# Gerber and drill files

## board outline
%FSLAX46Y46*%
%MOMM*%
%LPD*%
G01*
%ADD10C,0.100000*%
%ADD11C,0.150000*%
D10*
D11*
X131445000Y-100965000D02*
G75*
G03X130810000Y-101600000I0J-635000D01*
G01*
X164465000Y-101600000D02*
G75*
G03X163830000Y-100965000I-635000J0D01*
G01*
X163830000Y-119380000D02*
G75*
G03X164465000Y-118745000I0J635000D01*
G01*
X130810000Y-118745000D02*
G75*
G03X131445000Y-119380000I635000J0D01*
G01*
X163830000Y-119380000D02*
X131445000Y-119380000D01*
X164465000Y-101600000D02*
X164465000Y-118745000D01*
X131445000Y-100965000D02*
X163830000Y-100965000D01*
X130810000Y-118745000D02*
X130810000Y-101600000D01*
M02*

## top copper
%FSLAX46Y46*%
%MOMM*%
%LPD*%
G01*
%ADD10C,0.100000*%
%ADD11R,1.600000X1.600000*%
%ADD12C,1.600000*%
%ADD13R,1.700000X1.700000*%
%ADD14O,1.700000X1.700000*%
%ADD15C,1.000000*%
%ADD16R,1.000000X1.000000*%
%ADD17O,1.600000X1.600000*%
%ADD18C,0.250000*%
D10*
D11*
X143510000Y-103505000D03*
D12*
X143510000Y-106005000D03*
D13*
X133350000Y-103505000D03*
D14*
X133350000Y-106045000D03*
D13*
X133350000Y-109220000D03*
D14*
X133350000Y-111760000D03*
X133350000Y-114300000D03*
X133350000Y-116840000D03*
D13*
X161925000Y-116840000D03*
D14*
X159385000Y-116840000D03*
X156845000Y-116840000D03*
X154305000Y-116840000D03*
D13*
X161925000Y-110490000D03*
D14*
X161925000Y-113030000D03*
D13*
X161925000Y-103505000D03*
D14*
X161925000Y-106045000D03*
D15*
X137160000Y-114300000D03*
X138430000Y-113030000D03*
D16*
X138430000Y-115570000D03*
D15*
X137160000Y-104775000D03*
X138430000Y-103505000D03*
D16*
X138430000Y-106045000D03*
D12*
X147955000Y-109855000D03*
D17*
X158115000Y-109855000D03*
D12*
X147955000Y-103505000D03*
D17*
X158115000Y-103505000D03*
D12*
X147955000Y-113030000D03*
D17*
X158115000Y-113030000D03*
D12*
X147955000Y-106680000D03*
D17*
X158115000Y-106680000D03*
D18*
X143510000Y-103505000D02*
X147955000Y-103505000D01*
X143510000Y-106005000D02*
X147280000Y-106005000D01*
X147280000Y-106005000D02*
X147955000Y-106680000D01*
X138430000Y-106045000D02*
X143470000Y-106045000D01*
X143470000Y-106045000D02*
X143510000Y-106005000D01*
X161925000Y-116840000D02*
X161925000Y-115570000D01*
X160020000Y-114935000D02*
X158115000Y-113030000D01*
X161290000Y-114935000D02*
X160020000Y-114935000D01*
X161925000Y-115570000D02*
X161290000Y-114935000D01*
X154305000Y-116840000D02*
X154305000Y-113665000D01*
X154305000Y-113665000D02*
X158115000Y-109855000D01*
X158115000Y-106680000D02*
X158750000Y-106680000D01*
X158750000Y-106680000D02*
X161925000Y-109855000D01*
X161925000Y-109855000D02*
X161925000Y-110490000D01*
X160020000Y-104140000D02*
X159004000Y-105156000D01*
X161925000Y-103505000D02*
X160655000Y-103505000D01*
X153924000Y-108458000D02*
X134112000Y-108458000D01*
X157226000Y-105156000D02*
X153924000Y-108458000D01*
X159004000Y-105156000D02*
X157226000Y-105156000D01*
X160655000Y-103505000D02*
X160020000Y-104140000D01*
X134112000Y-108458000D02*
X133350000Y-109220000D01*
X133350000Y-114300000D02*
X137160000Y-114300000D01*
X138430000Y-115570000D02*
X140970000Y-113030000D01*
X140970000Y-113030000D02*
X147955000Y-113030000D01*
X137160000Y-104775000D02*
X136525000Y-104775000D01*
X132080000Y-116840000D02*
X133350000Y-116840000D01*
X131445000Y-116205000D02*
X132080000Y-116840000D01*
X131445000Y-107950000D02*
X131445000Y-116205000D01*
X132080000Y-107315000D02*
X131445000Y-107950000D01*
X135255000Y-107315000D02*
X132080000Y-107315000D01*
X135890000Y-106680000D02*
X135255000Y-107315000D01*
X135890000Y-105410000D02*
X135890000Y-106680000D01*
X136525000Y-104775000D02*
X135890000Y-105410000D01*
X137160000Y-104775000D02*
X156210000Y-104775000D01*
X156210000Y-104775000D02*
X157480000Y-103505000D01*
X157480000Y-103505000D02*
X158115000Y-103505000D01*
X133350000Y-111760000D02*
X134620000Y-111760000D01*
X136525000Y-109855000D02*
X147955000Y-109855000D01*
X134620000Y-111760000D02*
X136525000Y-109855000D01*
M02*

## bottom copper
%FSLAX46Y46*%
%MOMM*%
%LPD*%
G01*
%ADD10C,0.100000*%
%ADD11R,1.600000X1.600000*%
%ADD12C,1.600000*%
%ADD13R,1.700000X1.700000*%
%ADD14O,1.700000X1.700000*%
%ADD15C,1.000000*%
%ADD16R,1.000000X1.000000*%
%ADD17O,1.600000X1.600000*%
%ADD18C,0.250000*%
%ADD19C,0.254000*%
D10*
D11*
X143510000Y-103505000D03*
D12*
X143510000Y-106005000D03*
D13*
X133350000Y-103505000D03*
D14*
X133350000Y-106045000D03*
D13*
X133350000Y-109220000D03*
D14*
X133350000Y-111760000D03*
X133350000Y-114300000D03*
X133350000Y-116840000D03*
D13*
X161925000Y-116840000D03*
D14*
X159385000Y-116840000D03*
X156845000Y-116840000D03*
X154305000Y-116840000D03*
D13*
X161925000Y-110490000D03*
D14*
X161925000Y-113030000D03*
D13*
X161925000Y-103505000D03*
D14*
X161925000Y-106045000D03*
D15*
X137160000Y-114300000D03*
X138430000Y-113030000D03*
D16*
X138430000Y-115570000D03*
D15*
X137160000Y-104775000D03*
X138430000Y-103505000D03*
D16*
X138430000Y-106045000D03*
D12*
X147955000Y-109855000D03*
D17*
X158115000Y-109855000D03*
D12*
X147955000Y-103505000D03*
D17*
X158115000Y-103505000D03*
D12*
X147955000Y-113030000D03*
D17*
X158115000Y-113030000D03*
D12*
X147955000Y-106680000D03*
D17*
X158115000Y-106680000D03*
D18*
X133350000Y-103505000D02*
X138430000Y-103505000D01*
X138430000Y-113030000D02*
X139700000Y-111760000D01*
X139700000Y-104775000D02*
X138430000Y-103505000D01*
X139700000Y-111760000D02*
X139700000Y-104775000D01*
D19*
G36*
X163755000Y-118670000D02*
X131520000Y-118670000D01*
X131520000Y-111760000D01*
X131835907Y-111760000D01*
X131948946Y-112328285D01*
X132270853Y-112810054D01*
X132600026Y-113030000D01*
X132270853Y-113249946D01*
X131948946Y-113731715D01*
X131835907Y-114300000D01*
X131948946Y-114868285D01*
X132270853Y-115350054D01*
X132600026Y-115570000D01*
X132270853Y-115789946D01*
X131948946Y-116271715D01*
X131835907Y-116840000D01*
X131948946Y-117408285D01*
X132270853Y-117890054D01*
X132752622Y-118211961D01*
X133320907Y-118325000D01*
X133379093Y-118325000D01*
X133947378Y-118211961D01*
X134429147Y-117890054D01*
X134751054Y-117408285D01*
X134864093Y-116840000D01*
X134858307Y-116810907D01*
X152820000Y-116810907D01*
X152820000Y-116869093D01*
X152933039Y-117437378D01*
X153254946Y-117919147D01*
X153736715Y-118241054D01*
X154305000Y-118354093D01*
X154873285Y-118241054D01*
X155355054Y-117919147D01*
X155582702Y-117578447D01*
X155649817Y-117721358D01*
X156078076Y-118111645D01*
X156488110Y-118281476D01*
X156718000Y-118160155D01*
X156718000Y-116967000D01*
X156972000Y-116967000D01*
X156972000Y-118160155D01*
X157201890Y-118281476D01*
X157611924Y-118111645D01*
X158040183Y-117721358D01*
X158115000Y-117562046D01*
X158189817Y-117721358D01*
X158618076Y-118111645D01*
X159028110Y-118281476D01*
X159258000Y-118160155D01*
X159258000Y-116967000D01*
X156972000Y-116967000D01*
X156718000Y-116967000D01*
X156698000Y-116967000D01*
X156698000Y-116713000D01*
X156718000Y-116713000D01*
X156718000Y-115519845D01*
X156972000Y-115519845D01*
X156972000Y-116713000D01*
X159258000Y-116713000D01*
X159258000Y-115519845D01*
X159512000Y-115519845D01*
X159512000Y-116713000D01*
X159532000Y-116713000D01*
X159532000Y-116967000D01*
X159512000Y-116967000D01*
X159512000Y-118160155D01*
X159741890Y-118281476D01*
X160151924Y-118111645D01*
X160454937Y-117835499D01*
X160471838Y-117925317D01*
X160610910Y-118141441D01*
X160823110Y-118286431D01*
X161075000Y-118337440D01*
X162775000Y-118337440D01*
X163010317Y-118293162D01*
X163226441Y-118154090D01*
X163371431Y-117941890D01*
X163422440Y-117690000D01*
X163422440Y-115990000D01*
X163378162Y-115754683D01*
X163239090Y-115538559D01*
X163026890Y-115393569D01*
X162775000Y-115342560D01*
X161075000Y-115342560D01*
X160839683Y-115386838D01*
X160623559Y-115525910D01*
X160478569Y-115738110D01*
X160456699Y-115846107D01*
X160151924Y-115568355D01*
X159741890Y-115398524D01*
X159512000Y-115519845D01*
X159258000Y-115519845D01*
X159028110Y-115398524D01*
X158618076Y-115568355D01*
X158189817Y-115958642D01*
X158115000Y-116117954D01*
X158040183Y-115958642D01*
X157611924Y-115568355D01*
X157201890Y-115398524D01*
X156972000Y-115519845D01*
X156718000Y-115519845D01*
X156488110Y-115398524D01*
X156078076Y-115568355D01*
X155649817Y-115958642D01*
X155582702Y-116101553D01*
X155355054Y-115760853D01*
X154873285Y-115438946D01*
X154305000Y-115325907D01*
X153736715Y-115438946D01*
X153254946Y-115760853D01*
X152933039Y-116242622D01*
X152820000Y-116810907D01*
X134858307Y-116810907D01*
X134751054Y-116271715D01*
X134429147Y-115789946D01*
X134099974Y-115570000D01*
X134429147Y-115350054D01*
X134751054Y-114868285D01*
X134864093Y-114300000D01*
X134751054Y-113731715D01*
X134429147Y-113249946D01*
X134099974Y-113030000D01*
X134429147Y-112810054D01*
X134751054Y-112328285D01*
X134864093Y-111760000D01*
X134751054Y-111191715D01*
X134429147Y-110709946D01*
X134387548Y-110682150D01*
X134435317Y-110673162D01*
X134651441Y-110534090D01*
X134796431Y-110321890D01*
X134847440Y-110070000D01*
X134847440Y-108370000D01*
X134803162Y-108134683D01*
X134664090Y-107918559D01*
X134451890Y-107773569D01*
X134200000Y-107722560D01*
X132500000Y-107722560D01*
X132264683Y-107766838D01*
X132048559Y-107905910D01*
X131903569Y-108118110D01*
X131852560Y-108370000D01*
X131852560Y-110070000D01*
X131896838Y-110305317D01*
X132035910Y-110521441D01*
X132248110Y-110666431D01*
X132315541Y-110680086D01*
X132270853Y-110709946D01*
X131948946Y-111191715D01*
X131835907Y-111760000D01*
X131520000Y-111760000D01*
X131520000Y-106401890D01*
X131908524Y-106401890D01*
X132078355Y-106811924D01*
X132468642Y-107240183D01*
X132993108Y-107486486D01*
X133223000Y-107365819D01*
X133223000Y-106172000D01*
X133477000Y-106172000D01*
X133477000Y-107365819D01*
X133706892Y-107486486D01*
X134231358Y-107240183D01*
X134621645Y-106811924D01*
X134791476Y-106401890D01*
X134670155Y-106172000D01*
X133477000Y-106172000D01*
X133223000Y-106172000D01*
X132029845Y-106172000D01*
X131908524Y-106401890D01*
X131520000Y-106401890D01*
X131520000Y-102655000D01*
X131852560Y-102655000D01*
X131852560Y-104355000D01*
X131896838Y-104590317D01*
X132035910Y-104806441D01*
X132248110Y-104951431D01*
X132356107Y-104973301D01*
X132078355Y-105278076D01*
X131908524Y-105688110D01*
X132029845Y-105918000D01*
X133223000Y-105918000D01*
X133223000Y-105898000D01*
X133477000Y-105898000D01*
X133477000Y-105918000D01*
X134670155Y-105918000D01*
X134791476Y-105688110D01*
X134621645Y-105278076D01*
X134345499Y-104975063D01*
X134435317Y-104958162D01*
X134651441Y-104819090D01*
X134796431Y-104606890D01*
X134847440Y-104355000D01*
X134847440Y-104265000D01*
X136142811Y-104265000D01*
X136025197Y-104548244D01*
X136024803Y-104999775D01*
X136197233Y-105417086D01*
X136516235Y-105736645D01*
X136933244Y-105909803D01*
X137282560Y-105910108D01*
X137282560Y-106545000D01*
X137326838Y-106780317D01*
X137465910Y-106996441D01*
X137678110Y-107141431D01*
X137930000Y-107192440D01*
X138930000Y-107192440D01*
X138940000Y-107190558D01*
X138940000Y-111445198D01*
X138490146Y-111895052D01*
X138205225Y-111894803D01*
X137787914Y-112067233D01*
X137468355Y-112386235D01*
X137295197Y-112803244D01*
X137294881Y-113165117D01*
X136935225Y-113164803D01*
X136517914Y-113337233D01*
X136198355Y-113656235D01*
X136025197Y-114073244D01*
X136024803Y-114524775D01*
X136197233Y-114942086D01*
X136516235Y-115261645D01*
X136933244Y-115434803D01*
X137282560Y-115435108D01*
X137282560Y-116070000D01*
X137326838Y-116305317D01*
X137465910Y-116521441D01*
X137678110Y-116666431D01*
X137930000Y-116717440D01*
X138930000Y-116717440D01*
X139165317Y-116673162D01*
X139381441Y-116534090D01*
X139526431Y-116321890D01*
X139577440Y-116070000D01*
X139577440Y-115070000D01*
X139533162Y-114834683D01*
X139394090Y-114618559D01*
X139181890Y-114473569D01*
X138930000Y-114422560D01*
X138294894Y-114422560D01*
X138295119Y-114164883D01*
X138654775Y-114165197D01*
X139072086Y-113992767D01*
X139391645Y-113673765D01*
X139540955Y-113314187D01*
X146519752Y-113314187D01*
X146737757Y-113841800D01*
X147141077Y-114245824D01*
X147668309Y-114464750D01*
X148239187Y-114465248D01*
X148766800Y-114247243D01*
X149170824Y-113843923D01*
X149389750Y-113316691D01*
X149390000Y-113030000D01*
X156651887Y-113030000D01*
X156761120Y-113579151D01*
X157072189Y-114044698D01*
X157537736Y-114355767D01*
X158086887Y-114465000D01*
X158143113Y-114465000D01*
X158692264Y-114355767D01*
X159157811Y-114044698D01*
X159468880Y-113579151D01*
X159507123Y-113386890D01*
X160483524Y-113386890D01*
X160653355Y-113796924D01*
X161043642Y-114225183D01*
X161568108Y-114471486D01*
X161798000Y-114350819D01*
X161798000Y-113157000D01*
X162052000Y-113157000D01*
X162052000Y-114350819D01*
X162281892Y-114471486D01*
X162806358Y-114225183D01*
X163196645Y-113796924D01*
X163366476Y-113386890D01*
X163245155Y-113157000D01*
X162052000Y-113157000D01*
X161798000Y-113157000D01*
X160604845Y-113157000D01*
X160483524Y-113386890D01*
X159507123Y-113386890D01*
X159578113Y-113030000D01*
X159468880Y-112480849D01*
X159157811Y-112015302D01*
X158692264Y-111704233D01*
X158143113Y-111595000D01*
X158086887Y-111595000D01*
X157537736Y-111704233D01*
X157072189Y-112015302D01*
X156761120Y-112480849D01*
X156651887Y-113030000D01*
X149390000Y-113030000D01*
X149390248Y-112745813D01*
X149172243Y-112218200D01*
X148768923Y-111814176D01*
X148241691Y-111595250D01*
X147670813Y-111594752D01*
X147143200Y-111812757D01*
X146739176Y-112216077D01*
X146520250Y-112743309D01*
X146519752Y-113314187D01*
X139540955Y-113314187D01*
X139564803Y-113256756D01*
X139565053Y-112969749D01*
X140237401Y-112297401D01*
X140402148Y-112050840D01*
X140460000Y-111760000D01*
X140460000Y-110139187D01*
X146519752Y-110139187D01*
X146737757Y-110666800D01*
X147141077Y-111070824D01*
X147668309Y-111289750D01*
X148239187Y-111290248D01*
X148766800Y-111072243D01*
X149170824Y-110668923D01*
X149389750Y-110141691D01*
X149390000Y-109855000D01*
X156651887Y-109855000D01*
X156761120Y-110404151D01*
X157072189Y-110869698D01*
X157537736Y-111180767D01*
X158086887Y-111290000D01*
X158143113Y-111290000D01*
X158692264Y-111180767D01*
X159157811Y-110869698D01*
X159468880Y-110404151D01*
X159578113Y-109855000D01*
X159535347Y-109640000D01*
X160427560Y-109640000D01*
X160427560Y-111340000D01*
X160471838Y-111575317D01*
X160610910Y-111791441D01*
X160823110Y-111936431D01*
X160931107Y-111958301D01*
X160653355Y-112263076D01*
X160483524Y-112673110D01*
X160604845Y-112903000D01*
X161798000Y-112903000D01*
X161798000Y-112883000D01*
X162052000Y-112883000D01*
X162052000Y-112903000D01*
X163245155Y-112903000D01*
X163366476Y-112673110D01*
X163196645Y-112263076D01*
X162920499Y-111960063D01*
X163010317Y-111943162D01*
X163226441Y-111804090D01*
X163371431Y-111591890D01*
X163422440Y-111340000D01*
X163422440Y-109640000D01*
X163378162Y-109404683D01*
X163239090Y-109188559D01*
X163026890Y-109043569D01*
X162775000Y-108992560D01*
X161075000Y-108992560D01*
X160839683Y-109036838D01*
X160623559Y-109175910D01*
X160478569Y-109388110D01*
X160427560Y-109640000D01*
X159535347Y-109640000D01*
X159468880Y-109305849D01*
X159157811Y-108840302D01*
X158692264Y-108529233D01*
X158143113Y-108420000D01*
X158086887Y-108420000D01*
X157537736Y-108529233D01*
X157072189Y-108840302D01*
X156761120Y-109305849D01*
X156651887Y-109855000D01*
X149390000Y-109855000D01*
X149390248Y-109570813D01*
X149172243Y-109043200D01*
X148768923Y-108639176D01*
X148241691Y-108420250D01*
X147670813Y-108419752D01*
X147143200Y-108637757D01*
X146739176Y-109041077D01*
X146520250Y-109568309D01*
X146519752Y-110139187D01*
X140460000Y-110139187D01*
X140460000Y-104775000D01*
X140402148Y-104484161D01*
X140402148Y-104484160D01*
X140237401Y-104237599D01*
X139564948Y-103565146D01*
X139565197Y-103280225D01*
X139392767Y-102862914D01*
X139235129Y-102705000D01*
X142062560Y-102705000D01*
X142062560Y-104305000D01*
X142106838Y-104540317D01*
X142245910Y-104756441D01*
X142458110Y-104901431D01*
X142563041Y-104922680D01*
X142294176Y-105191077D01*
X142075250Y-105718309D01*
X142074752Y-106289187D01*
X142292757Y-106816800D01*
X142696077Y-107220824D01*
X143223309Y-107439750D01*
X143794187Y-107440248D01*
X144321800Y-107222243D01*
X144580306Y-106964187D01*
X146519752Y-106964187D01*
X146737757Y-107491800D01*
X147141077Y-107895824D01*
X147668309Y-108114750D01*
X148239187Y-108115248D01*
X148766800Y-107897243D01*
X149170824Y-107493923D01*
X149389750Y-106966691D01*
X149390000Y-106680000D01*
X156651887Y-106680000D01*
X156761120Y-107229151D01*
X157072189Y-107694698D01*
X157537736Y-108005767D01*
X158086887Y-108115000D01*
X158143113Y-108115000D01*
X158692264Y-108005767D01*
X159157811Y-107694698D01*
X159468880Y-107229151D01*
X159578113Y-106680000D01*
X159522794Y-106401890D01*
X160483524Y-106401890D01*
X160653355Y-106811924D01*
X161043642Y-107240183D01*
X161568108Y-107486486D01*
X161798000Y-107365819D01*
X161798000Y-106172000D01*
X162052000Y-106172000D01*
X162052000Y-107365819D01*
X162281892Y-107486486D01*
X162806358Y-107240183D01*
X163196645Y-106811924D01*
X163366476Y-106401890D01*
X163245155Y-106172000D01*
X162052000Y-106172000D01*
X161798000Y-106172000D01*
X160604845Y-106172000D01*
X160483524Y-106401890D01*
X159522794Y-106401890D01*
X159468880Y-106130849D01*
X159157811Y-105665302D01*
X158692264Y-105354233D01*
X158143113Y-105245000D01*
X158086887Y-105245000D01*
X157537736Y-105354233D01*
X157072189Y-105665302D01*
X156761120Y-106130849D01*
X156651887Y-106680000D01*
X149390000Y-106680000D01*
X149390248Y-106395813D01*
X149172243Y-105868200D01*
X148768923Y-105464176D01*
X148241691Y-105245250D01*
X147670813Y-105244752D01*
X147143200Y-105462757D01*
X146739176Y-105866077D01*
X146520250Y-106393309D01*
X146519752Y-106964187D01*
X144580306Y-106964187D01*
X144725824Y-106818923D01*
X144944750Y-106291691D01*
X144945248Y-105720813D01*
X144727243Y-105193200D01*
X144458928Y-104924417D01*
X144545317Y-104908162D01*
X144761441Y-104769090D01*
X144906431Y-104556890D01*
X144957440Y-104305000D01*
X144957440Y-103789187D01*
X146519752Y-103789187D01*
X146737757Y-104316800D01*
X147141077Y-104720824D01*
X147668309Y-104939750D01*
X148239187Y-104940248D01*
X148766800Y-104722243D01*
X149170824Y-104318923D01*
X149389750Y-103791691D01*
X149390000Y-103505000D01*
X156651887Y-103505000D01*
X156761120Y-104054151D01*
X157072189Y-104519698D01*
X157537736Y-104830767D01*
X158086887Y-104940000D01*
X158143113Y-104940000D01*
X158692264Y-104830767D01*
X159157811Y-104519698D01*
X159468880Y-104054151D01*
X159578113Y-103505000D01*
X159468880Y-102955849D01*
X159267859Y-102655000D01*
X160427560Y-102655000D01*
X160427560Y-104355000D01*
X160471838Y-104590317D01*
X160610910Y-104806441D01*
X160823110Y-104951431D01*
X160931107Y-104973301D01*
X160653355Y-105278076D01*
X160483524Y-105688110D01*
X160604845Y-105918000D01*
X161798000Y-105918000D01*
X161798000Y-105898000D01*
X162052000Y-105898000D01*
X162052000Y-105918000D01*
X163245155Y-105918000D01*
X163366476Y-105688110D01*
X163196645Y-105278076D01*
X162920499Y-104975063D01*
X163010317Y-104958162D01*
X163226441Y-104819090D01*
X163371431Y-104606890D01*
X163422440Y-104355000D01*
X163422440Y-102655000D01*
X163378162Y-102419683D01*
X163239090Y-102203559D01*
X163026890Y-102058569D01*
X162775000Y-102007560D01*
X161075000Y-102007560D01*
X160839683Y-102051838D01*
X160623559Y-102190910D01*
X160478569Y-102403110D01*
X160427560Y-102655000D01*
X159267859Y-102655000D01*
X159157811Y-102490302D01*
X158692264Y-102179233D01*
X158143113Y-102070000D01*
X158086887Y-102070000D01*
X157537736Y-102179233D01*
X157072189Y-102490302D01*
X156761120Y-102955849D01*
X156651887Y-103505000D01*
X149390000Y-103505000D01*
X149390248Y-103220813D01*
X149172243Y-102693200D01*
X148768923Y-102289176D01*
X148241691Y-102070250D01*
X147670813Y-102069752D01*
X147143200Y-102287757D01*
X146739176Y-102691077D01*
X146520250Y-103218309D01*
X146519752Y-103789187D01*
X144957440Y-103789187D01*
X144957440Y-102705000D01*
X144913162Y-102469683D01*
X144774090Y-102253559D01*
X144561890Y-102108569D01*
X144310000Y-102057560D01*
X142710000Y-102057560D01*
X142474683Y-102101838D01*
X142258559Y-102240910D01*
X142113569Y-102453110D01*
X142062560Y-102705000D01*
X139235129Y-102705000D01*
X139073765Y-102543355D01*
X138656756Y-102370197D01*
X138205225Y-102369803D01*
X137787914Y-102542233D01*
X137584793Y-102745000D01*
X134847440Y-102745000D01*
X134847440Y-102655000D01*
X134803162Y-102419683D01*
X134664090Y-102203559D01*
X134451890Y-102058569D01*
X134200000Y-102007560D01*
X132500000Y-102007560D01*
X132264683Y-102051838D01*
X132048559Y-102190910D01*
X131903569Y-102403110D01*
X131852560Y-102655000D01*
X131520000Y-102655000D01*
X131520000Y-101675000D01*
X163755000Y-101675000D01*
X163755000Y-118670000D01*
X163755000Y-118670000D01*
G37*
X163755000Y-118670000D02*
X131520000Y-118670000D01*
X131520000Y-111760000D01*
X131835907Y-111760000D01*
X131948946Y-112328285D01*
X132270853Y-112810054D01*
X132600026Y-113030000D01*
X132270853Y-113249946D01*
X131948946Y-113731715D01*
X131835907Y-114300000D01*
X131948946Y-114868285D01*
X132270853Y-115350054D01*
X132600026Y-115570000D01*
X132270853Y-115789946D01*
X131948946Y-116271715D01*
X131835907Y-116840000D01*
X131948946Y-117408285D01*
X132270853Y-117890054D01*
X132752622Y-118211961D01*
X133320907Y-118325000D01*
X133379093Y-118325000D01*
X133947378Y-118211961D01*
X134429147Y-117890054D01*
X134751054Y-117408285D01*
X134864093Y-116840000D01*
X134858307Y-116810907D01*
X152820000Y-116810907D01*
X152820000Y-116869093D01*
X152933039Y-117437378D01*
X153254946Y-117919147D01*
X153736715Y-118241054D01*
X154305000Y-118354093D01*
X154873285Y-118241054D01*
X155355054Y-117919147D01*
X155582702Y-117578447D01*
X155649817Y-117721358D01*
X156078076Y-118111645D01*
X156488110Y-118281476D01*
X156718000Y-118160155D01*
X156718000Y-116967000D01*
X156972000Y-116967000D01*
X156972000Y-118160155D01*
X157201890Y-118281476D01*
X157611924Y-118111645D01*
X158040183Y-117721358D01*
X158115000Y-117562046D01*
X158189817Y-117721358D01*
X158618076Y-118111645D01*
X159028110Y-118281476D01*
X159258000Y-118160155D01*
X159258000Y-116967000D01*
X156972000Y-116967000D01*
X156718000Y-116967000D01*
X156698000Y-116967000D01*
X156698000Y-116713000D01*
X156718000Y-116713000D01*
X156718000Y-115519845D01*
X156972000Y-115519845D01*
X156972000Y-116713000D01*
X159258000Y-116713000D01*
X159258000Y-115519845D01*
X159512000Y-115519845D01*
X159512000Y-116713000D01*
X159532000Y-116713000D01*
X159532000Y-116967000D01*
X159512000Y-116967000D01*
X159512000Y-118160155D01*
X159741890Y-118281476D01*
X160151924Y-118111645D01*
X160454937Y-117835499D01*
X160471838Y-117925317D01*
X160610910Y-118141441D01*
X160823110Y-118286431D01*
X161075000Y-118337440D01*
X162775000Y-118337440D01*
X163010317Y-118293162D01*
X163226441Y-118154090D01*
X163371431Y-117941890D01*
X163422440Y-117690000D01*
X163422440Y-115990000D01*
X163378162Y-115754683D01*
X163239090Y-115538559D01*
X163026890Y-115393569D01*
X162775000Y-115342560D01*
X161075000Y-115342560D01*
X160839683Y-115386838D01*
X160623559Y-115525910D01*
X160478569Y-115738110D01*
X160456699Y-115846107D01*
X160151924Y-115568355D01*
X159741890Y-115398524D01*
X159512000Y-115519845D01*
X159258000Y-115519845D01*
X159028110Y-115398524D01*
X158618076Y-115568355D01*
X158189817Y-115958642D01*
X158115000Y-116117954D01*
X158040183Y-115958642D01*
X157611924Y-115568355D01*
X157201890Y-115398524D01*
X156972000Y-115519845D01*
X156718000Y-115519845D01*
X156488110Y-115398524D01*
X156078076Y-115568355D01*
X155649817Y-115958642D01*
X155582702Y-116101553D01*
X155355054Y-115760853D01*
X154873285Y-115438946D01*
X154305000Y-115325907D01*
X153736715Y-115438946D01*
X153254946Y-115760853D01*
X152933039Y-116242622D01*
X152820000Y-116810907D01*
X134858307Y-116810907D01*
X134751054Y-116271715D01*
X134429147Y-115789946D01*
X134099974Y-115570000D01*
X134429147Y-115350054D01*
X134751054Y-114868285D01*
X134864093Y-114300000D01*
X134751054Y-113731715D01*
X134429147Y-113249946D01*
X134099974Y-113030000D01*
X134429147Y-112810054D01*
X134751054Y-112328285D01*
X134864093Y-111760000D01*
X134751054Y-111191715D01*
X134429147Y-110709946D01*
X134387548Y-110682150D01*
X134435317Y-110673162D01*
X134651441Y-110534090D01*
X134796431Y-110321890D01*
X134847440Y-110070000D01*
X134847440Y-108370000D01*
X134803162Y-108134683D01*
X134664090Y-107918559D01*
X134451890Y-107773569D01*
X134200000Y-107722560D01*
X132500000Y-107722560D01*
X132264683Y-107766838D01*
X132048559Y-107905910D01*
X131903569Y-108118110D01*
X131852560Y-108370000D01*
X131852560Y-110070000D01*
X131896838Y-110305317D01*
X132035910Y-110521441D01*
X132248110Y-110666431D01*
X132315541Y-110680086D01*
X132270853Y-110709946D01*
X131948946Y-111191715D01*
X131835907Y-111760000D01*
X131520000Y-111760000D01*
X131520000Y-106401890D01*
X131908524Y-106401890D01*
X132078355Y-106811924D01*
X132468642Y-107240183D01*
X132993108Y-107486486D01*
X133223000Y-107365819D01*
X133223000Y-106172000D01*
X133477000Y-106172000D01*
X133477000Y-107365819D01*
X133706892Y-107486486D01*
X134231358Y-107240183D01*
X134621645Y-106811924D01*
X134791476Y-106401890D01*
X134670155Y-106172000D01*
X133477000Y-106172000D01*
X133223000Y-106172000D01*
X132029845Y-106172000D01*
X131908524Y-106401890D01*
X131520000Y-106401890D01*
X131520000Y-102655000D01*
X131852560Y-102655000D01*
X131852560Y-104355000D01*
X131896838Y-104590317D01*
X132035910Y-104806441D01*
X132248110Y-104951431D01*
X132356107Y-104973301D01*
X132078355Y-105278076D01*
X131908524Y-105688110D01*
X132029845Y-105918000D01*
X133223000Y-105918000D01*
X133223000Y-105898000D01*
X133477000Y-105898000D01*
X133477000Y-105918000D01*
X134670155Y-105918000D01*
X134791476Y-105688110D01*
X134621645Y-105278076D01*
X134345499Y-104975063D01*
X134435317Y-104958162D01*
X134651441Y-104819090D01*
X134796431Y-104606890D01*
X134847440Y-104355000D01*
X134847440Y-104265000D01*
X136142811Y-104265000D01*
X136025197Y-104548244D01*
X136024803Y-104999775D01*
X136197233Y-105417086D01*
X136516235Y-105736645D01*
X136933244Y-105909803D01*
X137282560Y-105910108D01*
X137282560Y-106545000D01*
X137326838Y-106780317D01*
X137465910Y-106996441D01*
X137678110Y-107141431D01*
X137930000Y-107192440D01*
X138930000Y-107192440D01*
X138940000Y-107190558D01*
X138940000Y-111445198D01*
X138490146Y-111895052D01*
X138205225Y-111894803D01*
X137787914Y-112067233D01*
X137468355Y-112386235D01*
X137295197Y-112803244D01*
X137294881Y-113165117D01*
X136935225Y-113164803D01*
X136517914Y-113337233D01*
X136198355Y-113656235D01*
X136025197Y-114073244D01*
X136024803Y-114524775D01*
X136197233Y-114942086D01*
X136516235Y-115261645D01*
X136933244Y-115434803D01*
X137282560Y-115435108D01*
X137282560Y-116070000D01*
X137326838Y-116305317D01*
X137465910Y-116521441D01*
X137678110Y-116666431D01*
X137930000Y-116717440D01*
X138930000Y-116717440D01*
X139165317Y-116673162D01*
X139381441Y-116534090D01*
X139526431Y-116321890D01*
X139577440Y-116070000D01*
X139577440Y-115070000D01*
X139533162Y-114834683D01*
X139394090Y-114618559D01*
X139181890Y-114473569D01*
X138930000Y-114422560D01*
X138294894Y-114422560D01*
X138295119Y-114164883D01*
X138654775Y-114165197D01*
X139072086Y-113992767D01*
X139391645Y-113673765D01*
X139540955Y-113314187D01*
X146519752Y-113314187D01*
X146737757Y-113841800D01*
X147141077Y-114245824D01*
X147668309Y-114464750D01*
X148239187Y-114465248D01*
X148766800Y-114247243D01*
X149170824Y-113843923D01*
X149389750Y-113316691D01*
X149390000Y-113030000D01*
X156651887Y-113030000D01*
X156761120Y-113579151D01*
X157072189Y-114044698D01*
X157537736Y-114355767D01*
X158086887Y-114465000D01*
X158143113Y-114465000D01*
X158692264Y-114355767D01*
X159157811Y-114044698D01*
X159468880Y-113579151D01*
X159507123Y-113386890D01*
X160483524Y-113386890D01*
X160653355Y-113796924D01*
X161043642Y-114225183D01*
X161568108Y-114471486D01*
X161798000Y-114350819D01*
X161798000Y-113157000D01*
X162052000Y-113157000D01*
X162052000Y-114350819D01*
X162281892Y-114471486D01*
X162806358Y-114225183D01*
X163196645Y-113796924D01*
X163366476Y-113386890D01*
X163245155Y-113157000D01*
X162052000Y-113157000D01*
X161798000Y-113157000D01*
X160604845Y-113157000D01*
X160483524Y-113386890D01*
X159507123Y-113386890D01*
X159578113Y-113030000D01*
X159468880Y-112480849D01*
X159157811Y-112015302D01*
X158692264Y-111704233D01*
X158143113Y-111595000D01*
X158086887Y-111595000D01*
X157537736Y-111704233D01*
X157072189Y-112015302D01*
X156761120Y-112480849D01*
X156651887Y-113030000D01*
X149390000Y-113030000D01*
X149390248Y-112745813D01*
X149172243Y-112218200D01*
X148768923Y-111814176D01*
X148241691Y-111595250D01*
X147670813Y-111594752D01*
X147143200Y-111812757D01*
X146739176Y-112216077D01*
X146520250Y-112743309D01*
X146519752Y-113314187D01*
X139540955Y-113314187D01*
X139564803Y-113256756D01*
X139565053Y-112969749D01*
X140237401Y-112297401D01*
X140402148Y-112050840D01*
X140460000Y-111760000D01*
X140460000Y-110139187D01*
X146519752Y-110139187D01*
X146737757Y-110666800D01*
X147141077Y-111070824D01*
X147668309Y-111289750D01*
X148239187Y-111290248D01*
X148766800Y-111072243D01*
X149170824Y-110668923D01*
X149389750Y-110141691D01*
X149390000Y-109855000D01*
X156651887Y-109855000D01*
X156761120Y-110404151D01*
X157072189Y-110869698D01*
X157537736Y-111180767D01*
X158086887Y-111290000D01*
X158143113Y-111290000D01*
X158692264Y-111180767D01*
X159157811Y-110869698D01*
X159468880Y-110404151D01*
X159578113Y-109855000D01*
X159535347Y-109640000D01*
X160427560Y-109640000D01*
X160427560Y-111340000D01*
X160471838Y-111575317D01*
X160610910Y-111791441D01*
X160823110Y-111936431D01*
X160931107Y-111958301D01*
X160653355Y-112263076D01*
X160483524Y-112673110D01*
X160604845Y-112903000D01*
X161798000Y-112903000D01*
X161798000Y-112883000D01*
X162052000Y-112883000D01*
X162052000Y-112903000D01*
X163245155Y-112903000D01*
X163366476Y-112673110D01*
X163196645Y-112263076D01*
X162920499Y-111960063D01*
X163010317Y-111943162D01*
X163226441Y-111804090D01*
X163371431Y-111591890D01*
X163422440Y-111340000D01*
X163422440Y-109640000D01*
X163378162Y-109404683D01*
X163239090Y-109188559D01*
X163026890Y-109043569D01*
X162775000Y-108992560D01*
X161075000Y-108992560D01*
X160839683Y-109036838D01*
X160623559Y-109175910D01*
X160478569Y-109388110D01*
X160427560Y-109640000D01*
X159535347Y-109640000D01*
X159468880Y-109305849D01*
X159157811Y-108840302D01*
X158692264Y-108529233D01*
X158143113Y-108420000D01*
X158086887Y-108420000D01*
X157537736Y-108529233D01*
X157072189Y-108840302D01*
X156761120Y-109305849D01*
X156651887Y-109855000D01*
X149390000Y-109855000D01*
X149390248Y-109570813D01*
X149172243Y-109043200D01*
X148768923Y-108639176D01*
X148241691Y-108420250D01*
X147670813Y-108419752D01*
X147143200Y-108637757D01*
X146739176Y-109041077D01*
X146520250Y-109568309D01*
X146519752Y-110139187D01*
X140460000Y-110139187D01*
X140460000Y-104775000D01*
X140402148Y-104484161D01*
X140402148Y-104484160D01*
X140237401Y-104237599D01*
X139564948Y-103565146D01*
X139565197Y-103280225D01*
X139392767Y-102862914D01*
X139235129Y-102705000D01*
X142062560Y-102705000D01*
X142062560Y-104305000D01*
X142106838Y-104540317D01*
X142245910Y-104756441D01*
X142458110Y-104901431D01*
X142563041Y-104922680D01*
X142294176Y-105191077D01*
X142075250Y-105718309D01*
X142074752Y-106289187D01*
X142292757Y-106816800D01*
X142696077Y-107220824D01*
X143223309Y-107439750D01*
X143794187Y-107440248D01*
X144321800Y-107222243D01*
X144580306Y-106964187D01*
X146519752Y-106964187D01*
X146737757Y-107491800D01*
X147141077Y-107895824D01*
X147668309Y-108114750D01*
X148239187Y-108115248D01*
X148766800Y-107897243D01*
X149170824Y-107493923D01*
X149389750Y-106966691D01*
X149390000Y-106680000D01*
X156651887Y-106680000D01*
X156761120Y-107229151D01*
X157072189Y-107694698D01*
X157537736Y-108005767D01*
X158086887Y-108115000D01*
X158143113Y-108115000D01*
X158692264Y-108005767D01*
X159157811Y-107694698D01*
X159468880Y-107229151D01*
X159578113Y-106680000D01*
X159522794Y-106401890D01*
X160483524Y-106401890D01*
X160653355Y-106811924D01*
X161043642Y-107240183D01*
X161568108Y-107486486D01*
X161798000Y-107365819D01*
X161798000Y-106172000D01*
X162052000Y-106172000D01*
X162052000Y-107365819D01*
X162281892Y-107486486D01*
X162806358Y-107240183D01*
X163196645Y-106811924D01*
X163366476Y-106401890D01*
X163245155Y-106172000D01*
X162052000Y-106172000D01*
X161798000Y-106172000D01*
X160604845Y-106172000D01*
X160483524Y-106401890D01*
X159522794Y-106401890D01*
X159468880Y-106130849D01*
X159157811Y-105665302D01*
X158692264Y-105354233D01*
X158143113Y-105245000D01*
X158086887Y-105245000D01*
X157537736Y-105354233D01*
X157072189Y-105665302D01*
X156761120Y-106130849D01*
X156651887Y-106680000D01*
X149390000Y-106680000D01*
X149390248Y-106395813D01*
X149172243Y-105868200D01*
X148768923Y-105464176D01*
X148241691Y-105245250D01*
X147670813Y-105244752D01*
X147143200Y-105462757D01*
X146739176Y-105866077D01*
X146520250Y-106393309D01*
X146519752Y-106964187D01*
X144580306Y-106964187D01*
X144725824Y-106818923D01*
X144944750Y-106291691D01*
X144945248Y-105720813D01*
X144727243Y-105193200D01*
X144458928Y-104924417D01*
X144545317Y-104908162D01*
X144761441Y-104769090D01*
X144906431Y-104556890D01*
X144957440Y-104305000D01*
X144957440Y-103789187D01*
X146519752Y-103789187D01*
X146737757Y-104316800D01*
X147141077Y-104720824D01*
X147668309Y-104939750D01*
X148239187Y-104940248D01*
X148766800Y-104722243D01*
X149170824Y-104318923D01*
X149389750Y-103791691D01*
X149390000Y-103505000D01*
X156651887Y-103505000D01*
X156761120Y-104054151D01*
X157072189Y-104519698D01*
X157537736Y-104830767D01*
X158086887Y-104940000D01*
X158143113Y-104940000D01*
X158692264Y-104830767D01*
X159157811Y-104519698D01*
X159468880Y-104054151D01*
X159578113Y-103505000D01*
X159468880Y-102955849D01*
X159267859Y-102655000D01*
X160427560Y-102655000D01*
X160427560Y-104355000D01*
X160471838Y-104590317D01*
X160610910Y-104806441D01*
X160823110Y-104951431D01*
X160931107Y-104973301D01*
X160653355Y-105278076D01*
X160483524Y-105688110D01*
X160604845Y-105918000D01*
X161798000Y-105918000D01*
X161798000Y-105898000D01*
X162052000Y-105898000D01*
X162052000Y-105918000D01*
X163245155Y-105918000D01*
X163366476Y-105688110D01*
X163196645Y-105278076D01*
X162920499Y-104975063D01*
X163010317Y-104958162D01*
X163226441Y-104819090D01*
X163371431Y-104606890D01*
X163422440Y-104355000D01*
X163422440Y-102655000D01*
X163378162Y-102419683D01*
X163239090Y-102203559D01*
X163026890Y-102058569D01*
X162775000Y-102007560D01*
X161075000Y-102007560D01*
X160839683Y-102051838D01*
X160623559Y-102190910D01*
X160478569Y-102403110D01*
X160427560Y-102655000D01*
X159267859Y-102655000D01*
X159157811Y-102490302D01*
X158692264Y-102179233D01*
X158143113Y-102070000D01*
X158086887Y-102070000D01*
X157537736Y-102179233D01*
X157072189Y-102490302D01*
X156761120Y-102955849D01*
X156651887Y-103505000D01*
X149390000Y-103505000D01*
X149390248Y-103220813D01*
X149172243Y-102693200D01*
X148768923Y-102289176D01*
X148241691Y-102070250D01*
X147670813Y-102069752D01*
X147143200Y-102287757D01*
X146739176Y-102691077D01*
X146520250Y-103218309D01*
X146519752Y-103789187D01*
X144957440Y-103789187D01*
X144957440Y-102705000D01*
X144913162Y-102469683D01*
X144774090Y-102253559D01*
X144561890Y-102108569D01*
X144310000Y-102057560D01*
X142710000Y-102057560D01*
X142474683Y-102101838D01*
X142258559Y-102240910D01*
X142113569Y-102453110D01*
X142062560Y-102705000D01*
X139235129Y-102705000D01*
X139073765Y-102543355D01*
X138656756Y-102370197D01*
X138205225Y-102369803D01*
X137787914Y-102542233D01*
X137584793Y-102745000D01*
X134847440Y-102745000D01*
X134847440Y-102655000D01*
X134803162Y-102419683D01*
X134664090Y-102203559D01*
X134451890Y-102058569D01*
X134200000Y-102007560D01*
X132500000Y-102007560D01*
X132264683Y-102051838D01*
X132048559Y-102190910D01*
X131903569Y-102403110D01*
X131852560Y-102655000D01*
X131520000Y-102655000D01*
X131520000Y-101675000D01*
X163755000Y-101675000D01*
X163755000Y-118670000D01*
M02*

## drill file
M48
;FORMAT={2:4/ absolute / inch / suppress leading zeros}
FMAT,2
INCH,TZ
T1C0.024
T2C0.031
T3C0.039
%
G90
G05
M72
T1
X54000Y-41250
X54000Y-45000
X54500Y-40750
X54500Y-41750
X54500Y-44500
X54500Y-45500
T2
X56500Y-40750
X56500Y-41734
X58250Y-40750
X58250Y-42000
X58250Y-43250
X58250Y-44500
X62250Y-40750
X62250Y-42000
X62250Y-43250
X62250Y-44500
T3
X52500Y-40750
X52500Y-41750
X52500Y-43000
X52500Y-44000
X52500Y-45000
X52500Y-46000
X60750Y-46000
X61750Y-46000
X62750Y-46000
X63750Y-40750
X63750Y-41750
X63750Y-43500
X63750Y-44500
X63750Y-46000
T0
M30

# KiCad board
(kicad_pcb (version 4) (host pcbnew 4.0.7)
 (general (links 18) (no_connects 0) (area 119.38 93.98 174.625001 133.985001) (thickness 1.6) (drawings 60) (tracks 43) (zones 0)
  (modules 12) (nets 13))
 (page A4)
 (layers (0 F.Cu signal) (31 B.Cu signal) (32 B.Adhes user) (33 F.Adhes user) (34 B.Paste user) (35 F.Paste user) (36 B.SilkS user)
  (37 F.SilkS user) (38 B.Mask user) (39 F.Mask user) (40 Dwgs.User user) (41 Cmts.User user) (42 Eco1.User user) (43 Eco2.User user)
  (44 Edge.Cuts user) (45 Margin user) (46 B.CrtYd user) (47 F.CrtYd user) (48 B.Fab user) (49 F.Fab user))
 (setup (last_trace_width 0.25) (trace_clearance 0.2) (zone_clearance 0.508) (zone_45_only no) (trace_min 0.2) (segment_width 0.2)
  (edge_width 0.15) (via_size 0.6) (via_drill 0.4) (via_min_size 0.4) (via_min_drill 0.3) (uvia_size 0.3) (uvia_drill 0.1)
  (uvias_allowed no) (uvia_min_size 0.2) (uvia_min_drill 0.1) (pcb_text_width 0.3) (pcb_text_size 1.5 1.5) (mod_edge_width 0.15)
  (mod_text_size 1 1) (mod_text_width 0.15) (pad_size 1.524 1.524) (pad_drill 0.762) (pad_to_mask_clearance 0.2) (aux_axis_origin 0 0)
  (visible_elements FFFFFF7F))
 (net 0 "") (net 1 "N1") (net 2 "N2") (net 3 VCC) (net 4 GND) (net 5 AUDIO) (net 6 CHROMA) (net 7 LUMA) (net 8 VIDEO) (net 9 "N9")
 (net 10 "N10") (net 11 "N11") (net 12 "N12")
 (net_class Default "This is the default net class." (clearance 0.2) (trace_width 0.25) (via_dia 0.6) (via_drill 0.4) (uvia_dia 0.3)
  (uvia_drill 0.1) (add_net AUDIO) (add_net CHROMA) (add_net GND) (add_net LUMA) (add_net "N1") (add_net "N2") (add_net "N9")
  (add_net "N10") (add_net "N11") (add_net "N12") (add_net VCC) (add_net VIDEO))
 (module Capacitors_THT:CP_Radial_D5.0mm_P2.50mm (layer F.Cu) (at 143.51 103.505 270)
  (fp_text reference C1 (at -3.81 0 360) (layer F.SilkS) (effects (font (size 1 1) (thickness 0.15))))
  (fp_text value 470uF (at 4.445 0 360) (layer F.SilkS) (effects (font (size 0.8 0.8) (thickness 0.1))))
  (pad 1 thru_hole rect (at 0 0 270) (size 1.6 1.6) (drill 0.8) (layers *.Cu *.Mask) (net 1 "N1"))
  (pad 2 thru_hole circle (at 2.5 0 270) (size 1.6 1.6) (drill 0.8) (layers *.Cu *.Mask) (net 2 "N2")))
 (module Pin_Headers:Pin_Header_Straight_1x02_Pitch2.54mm (layer F.Cu) (at 133.35 103.505)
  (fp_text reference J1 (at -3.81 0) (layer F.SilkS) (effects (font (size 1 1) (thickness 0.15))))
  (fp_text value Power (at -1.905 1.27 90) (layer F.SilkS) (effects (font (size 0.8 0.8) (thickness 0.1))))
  (pad 1 thru_hole rect (at 0 0) (size 1.7 1.7) (drill 1) (layers *.Cu *.Mask) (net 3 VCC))
  (pad 2 thru_hole oval (at 0 2.54) (size 1.7 1.7) (drill 1) (layers *.Cu *.Mask) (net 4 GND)))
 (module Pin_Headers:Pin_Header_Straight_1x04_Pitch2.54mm (layer F.Cu) (at 133.35 109.22)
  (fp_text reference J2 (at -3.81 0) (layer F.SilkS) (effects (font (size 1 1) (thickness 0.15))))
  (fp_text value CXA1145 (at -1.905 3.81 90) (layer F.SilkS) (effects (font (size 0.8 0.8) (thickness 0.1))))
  (pad 1 thru_hole rect (at 0 0) (size 1.7 1.7) (drill 1) (layers *.Cu *.Mask) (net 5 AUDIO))
  (pad 2 thru_hole oval (at 0 2.54) (size 1.7 1.7) (drill 1) (layers *.Cu *.Mask) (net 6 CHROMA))
  (pad 3 thru_hole oval (at 0 5.08) (size 1.7 1.7) (drill 1) (layers *.Cu *.Mask) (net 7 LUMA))
  (pad 4 thru_hole oval (at 0 7.62) (size 1.7 1.7) (drill 1) (layers *.Cu *.Mask) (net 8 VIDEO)))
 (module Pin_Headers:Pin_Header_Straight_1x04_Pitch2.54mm (layer F.Cu) (at 161.925 116.84 270)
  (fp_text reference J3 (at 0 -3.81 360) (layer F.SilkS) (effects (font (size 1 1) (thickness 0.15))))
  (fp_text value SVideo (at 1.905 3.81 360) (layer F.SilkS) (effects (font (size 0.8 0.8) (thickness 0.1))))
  (pad 1 thru_hole rect (at 0 0 270) (size 1.7 1.7) (drill 1) (layers *.Cu *.Mask) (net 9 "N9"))
  (pad 2 thru_hole oval (at 0 2.54 270) (size 1.7 1.7) (drill 1) (layers *.Cu *.Mask) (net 4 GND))
  (pad 3 thru_hole oval (at 0 5.08 270) (size 1.7 1.7) (drill 1) (layers *.Cu *.Mask) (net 4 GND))
  (pad 4 thru_hole oval (at 0 7.62 270) (size 1.7 1.7) (drill 1) (layers *.Cu *.Mask) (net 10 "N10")))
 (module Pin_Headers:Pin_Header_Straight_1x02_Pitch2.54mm (layer F.Cu) (at 161.925 110.49)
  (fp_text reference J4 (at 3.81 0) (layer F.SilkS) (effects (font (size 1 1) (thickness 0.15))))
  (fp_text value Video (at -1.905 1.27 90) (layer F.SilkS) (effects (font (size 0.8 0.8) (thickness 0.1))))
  (pad 1 thru_hole rect (at 0 0) (size 1.7 1.7) (drill 1) (layers *.Cu *.Mask) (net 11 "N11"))
  (pad 2 thru_hole oval (at 0 2.54) (size 1.7 1.7) (drill 1) (layers *.Cu *.Mask) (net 4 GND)))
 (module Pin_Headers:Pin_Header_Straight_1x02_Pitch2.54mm (layer F.Cu) (at 161.925 103.505)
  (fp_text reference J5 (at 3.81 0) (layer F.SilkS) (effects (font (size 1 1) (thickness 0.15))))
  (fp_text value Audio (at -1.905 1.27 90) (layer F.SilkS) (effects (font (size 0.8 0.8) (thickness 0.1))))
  (pad 1 thru_hole rect (at 0 0) (size 1.7 1.7) (drill 1) (layers *.Cu *.Mask) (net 5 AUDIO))
  (pad 2 thru_hole oval (at 0 2.54) (size 1.7 1.7) (drill 1) (layers *.Cu *.Mask) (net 4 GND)))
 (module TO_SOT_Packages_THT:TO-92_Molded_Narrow (layer F.Cu) (at 138.43 115.57 90)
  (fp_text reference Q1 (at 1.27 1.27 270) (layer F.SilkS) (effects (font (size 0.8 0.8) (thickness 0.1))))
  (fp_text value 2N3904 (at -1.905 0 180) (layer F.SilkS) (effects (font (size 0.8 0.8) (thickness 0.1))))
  (pad 2 thru_hole circle (at 1.27 -1.27 180) (size 1 1) (drill 0.6) (layers *.Cu *.Mask) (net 7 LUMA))
  (pad 3 thru_hole circle (at 2.54 0 180) (size 1 1) (drill 0.6) (layers *.Cu *.Mask) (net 3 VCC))
  (pad 1 thru_hole rect (at 0 0 180) (size 1 1) (drill 0.6) (layers *.Cu *.Mask) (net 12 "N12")))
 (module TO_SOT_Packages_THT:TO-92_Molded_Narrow (layer F.Cu) (at 138.43 106.045 90)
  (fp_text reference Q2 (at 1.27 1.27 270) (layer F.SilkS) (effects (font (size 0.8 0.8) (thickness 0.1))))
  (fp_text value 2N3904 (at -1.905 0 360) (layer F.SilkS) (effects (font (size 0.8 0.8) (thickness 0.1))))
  (pad 2 thru_hole circle (at 1.27 -1.27 180) (size 1 1) (drill 0.6) (layers *.Cu *.Mask) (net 8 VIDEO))
  (pad 3 thru_hole circle (at 2.54 0 180) (size 1 1) (drill 0.6) (layers *.Cu *.Mask) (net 3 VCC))
  (pad 1 thru_hole rect (at 0 0 180) (size 1 1) (drill 0.6) (layers *.Cu *.Mask) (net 2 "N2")))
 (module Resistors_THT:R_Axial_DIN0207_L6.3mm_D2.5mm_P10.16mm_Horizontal (layer F.Cu) (at 147.955 109.855)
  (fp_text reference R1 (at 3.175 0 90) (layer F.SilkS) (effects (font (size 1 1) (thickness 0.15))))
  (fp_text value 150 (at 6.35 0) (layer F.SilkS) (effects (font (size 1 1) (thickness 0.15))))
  (pad 1 thru_hole circle (at 0 0) (size 1.6 1.6) (drill 0.8) (layers *.Cu *.Mask) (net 6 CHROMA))
  (pad 2 thru_hole oval (at 10.16 0) (size 1.6 1.6) (drill 0.8) (layers *.Cu *.Mask) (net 10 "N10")))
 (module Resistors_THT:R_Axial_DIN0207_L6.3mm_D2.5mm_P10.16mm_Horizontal (layer F.Cu) (at 147.955 103.505)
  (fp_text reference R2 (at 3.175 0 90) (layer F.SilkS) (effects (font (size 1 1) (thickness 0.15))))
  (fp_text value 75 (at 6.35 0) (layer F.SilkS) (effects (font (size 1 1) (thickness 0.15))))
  (pad 1 thru_hole circle (at 0 0) (size 1.6 1.6) (drill 0.8) (layers *.Cu *.Mask) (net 1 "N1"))
  (pad 2 thru_hole oval (at 10.16 0) (size 1.6 1.6) (drill 0.8) (layers *.Cu *.Mask) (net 8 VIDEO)))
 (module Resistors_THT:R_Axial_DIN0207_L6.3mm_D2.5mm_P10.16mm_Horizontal (layer F.Cu) (at 147.955 113.03)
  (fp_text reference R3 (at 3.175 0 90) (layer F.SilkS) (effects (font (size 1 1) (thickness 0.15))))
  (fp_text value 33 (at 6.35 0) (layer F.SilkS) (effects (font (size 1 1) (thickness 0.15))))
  (pad 1 thru_hole circle (at 0 0) (size 1.6 1.6) (drill 0.8) (layers *.Cu *.Mask) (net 12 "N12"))
  (pad 2 thru_hole oval (at 10.16 0) (size 1.6 1.6) (drill 0.8) (layers *.Cu *.Mask) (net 9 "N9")))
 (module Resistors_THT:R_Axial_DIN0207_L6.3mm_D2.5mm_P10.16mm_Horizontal (layer F.Cu) (at 147.955 106.68)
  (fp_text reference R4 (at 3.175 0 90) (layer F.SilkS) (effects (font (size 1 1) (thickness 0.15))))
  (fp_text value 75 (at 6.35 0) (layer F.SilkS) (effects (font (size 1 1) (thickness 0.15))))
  (pad 1 thru_hole circle (at 0 0) (size 1.6 1.6) (drill 0.8) (layers *.Cu *.Mask) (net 2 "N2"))
  (pad 2 thru_hole oval (at 10.16 0) (size 1.6 1.6) (drill 0.8) (layers *.Cu *.Mask) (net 11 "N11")))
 (gr_arc (start 131.445 101.6) (end 130.81 101.6) (angle 90) (layer Edge.Cuts) (width 0.15))
 (gr_arc (start 163.83 101.6) (end 163.83 100.965) (angle 90) (layer Edge.Cuts) (width 0.15))
 (gr_arc (start 163.83 118.745) (end 164.465 118.745) (angle 90) (layer Edge.Cuts) (width 0.15))
 (gr_arc (start 131.445 118.745) (end 131.445 119.38) (angle 90) (layer Edge.Cuts) (width 0.15))
 (gr_line (start 163.83 119.38) (end 131.445 119.38) (angle 90) (layer Edge.Cuts) (width 0.15))
 (gr_line (start 164.465 101.6) (end 164.465 118.745) (angle 90) (layer Edge.Cuts) (width 0.15))
 (gr_line (start 131.445 100.965) (end 163.83 100.965) (angle 90) (layer Edge.Cuts) (width 0.15))
 (gr_line (start 130.81 118.745) (end 130.81 101.6) (angle 90) (layer Edge.Cuts) (width 0.15))
 (segment (start 143.51 103.505) (end 147.955 103.505) (width 0.25) (layer F.Cu) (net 1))
 (segment (start 143.51 106.005) (end 147.28 106.005) (width 0.25) (layer F.Cu) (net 2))
 (segment (start 147.28 106.005) (end 147.955 106.68) (width 0.25) (layer F.Cu) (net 2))
 (segment (start 138.43 106.045) (end 143.47 106.045) (width 0.25) (layer F.Cu) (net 2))
 (segment (start 143.47 106.045) (end 143.51 106.005) (width 0.25) (layer F.Cu) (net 2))
 (segment (start 133.35 103.505) (end 138.43 103.505) (width 0.25) (layer B.Cu) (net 3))
 (segment (start 138.43 113.03) (end 139.7 111.76) (width 0.25) (layer B.Cu) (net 3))
 (segment (start 139.7 104.775) (end 138.43 103.505) (width 0.25) (layer B.Cu) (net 3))
 (segment (start 139.7 111.76) (end 139.7 104.775) (width 0.25) (layer B.Cu) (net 3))
 (segment (start 161.925 116.84) (end 161.925 115.57) (width 0.25) (layer F.Cu) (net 9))
 (segment (start 160.02 114.935) (end 158.115 113.03) (width 0.25) (layer F.Cu) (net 9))
 (segment (start 161.29 114.935) (end 160.02 114.935) (width 0.25) (layer F.Cu) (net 9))
 (segment (start 161.925 115.57) (end 161.29 114.935) (width 0.25) (layer F.Cu) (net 9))
 (segment (start 154.305 116.84) (end 154.305 113.665) (width 0.25) (layer F.Cu) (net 10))
 (segment (start 154.305 113.665) (end 158.115 109.855) (width 0.25) (layer F.Cu) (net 10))
 (segment (start 158.115 106.68) (end 158.75 106.68) (width 0.25) (layer F.Cu) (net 11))
 (segment (start 158.75 106.68) (end 161.925 109.855) (width 0.25) (layer F.Cu) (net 11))
 (segment (start 161.925 109.855) (end 161.925 110.49) (width 0.25) (layer F.Cu) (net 11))
 (segment (start 160.02 104.14) (end 159.004 105.156) (width 0.25) (layer F.Cu) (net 5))
 (segment (start 161.925 103.505) (end 160.655 103.505) (width 0.25) (layer F.Cu) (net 5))
 (segment (start 153.924 108.458) (end 134.112 108.458) (width 0.25) (layer F.Cu) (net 5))
 (segment (start 157.226 105.156) (end 153.924 108.458) (width 0.25) (layer F.Cu) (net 5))
 (segment (start 159.004 105.156) (end 157.226 105.156) (width 0.25) (layer F.Cu) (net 5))
 (segment (start 160.655 103.505) (end 160.02 104.14) (width 0.25) (layer F.Cu) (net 5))
 (segment (start 134.112 108.458) (end 133.35 109.22) (width 0.25) (layer F.Cu) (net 5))
 (segment (start 133.35 114.3) (end 137.16 114.3) (width 0.25) (layer F.Cu) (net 7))
 (segment (start 138.43 115.57) (end 140.97 113.03) (width 0.25) (layer F.Cu) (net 12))
 (segment (start 140.97 113.03) (end 147.955 113.03) (width 0.25) (layer F.Cu) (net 12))
 (segment (start 137.16 104.775) (end 136.525 104.775) (width 0.25) (layer F.Cu) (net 8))
 (segment (start 132.08 116.84) (end 133.35 116.84) (width 0.25) (layer F.Cu) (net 8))
 (segment (start 131.445 116.205) (end 132.08 116.84) (width 0.25) (layer F.Cu) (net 8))
 (segment (start 131.445 107.95) (end 131.445 116.205) (width 0.25) (layer F.Cu) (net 8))
 (segment (start 132.08 107.315) (end 131.445 107.95) (width 0.25) (layer F.Cu) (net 8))
 (segment (start 135.255 107.315) (end 132.08 107.315) (width 0.25) (layer F.Cu) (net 8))
 (segment (start 135.89 106.68) (end 135.255 107.315) (width 0.25) (layer F.Cu) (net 8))
 (segment (start 135.89 105.41) (end 135.89 106.68) (width 0.25) (layer F.Cu) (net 8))
 (segment (start 136.525 104.775) (end 135.89 105.41) (width 0.25) (layer F.Cu) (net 8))
 (segment (start 137.16 104.775) (end 156.21 104.775) (width 0.25) (layer F.Cu) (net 8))
 (segment (start 156.21 104.775) (end 157.48 103.505) (width 0.25) (layer F.Cu) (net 8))
 (segment (start 157.48 103.505) (end 158.115 103.505) (width 0.25) (layer F.Cu) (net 8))
 (segment (start 133.35 111.76) (end 134.62 111.76) (width 0.25) (layer F.Cu) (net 6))
 (segment (start 136.525 109.855) (end 147.955 109.855) (width 0.25) (layer F.Cu) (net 6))
 (segment (start 134.62 111.76) (end 136.525 109.855) (width 0.25) (layer F.Cu) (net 6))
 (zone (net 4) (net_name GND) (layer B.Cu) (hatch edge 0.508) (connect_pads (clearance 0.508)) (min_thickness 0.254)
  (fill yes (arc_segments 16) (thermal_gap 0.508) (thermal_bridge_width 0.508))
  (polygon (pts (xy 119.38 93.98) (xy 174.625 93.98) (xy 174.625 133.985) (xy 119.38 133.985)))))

